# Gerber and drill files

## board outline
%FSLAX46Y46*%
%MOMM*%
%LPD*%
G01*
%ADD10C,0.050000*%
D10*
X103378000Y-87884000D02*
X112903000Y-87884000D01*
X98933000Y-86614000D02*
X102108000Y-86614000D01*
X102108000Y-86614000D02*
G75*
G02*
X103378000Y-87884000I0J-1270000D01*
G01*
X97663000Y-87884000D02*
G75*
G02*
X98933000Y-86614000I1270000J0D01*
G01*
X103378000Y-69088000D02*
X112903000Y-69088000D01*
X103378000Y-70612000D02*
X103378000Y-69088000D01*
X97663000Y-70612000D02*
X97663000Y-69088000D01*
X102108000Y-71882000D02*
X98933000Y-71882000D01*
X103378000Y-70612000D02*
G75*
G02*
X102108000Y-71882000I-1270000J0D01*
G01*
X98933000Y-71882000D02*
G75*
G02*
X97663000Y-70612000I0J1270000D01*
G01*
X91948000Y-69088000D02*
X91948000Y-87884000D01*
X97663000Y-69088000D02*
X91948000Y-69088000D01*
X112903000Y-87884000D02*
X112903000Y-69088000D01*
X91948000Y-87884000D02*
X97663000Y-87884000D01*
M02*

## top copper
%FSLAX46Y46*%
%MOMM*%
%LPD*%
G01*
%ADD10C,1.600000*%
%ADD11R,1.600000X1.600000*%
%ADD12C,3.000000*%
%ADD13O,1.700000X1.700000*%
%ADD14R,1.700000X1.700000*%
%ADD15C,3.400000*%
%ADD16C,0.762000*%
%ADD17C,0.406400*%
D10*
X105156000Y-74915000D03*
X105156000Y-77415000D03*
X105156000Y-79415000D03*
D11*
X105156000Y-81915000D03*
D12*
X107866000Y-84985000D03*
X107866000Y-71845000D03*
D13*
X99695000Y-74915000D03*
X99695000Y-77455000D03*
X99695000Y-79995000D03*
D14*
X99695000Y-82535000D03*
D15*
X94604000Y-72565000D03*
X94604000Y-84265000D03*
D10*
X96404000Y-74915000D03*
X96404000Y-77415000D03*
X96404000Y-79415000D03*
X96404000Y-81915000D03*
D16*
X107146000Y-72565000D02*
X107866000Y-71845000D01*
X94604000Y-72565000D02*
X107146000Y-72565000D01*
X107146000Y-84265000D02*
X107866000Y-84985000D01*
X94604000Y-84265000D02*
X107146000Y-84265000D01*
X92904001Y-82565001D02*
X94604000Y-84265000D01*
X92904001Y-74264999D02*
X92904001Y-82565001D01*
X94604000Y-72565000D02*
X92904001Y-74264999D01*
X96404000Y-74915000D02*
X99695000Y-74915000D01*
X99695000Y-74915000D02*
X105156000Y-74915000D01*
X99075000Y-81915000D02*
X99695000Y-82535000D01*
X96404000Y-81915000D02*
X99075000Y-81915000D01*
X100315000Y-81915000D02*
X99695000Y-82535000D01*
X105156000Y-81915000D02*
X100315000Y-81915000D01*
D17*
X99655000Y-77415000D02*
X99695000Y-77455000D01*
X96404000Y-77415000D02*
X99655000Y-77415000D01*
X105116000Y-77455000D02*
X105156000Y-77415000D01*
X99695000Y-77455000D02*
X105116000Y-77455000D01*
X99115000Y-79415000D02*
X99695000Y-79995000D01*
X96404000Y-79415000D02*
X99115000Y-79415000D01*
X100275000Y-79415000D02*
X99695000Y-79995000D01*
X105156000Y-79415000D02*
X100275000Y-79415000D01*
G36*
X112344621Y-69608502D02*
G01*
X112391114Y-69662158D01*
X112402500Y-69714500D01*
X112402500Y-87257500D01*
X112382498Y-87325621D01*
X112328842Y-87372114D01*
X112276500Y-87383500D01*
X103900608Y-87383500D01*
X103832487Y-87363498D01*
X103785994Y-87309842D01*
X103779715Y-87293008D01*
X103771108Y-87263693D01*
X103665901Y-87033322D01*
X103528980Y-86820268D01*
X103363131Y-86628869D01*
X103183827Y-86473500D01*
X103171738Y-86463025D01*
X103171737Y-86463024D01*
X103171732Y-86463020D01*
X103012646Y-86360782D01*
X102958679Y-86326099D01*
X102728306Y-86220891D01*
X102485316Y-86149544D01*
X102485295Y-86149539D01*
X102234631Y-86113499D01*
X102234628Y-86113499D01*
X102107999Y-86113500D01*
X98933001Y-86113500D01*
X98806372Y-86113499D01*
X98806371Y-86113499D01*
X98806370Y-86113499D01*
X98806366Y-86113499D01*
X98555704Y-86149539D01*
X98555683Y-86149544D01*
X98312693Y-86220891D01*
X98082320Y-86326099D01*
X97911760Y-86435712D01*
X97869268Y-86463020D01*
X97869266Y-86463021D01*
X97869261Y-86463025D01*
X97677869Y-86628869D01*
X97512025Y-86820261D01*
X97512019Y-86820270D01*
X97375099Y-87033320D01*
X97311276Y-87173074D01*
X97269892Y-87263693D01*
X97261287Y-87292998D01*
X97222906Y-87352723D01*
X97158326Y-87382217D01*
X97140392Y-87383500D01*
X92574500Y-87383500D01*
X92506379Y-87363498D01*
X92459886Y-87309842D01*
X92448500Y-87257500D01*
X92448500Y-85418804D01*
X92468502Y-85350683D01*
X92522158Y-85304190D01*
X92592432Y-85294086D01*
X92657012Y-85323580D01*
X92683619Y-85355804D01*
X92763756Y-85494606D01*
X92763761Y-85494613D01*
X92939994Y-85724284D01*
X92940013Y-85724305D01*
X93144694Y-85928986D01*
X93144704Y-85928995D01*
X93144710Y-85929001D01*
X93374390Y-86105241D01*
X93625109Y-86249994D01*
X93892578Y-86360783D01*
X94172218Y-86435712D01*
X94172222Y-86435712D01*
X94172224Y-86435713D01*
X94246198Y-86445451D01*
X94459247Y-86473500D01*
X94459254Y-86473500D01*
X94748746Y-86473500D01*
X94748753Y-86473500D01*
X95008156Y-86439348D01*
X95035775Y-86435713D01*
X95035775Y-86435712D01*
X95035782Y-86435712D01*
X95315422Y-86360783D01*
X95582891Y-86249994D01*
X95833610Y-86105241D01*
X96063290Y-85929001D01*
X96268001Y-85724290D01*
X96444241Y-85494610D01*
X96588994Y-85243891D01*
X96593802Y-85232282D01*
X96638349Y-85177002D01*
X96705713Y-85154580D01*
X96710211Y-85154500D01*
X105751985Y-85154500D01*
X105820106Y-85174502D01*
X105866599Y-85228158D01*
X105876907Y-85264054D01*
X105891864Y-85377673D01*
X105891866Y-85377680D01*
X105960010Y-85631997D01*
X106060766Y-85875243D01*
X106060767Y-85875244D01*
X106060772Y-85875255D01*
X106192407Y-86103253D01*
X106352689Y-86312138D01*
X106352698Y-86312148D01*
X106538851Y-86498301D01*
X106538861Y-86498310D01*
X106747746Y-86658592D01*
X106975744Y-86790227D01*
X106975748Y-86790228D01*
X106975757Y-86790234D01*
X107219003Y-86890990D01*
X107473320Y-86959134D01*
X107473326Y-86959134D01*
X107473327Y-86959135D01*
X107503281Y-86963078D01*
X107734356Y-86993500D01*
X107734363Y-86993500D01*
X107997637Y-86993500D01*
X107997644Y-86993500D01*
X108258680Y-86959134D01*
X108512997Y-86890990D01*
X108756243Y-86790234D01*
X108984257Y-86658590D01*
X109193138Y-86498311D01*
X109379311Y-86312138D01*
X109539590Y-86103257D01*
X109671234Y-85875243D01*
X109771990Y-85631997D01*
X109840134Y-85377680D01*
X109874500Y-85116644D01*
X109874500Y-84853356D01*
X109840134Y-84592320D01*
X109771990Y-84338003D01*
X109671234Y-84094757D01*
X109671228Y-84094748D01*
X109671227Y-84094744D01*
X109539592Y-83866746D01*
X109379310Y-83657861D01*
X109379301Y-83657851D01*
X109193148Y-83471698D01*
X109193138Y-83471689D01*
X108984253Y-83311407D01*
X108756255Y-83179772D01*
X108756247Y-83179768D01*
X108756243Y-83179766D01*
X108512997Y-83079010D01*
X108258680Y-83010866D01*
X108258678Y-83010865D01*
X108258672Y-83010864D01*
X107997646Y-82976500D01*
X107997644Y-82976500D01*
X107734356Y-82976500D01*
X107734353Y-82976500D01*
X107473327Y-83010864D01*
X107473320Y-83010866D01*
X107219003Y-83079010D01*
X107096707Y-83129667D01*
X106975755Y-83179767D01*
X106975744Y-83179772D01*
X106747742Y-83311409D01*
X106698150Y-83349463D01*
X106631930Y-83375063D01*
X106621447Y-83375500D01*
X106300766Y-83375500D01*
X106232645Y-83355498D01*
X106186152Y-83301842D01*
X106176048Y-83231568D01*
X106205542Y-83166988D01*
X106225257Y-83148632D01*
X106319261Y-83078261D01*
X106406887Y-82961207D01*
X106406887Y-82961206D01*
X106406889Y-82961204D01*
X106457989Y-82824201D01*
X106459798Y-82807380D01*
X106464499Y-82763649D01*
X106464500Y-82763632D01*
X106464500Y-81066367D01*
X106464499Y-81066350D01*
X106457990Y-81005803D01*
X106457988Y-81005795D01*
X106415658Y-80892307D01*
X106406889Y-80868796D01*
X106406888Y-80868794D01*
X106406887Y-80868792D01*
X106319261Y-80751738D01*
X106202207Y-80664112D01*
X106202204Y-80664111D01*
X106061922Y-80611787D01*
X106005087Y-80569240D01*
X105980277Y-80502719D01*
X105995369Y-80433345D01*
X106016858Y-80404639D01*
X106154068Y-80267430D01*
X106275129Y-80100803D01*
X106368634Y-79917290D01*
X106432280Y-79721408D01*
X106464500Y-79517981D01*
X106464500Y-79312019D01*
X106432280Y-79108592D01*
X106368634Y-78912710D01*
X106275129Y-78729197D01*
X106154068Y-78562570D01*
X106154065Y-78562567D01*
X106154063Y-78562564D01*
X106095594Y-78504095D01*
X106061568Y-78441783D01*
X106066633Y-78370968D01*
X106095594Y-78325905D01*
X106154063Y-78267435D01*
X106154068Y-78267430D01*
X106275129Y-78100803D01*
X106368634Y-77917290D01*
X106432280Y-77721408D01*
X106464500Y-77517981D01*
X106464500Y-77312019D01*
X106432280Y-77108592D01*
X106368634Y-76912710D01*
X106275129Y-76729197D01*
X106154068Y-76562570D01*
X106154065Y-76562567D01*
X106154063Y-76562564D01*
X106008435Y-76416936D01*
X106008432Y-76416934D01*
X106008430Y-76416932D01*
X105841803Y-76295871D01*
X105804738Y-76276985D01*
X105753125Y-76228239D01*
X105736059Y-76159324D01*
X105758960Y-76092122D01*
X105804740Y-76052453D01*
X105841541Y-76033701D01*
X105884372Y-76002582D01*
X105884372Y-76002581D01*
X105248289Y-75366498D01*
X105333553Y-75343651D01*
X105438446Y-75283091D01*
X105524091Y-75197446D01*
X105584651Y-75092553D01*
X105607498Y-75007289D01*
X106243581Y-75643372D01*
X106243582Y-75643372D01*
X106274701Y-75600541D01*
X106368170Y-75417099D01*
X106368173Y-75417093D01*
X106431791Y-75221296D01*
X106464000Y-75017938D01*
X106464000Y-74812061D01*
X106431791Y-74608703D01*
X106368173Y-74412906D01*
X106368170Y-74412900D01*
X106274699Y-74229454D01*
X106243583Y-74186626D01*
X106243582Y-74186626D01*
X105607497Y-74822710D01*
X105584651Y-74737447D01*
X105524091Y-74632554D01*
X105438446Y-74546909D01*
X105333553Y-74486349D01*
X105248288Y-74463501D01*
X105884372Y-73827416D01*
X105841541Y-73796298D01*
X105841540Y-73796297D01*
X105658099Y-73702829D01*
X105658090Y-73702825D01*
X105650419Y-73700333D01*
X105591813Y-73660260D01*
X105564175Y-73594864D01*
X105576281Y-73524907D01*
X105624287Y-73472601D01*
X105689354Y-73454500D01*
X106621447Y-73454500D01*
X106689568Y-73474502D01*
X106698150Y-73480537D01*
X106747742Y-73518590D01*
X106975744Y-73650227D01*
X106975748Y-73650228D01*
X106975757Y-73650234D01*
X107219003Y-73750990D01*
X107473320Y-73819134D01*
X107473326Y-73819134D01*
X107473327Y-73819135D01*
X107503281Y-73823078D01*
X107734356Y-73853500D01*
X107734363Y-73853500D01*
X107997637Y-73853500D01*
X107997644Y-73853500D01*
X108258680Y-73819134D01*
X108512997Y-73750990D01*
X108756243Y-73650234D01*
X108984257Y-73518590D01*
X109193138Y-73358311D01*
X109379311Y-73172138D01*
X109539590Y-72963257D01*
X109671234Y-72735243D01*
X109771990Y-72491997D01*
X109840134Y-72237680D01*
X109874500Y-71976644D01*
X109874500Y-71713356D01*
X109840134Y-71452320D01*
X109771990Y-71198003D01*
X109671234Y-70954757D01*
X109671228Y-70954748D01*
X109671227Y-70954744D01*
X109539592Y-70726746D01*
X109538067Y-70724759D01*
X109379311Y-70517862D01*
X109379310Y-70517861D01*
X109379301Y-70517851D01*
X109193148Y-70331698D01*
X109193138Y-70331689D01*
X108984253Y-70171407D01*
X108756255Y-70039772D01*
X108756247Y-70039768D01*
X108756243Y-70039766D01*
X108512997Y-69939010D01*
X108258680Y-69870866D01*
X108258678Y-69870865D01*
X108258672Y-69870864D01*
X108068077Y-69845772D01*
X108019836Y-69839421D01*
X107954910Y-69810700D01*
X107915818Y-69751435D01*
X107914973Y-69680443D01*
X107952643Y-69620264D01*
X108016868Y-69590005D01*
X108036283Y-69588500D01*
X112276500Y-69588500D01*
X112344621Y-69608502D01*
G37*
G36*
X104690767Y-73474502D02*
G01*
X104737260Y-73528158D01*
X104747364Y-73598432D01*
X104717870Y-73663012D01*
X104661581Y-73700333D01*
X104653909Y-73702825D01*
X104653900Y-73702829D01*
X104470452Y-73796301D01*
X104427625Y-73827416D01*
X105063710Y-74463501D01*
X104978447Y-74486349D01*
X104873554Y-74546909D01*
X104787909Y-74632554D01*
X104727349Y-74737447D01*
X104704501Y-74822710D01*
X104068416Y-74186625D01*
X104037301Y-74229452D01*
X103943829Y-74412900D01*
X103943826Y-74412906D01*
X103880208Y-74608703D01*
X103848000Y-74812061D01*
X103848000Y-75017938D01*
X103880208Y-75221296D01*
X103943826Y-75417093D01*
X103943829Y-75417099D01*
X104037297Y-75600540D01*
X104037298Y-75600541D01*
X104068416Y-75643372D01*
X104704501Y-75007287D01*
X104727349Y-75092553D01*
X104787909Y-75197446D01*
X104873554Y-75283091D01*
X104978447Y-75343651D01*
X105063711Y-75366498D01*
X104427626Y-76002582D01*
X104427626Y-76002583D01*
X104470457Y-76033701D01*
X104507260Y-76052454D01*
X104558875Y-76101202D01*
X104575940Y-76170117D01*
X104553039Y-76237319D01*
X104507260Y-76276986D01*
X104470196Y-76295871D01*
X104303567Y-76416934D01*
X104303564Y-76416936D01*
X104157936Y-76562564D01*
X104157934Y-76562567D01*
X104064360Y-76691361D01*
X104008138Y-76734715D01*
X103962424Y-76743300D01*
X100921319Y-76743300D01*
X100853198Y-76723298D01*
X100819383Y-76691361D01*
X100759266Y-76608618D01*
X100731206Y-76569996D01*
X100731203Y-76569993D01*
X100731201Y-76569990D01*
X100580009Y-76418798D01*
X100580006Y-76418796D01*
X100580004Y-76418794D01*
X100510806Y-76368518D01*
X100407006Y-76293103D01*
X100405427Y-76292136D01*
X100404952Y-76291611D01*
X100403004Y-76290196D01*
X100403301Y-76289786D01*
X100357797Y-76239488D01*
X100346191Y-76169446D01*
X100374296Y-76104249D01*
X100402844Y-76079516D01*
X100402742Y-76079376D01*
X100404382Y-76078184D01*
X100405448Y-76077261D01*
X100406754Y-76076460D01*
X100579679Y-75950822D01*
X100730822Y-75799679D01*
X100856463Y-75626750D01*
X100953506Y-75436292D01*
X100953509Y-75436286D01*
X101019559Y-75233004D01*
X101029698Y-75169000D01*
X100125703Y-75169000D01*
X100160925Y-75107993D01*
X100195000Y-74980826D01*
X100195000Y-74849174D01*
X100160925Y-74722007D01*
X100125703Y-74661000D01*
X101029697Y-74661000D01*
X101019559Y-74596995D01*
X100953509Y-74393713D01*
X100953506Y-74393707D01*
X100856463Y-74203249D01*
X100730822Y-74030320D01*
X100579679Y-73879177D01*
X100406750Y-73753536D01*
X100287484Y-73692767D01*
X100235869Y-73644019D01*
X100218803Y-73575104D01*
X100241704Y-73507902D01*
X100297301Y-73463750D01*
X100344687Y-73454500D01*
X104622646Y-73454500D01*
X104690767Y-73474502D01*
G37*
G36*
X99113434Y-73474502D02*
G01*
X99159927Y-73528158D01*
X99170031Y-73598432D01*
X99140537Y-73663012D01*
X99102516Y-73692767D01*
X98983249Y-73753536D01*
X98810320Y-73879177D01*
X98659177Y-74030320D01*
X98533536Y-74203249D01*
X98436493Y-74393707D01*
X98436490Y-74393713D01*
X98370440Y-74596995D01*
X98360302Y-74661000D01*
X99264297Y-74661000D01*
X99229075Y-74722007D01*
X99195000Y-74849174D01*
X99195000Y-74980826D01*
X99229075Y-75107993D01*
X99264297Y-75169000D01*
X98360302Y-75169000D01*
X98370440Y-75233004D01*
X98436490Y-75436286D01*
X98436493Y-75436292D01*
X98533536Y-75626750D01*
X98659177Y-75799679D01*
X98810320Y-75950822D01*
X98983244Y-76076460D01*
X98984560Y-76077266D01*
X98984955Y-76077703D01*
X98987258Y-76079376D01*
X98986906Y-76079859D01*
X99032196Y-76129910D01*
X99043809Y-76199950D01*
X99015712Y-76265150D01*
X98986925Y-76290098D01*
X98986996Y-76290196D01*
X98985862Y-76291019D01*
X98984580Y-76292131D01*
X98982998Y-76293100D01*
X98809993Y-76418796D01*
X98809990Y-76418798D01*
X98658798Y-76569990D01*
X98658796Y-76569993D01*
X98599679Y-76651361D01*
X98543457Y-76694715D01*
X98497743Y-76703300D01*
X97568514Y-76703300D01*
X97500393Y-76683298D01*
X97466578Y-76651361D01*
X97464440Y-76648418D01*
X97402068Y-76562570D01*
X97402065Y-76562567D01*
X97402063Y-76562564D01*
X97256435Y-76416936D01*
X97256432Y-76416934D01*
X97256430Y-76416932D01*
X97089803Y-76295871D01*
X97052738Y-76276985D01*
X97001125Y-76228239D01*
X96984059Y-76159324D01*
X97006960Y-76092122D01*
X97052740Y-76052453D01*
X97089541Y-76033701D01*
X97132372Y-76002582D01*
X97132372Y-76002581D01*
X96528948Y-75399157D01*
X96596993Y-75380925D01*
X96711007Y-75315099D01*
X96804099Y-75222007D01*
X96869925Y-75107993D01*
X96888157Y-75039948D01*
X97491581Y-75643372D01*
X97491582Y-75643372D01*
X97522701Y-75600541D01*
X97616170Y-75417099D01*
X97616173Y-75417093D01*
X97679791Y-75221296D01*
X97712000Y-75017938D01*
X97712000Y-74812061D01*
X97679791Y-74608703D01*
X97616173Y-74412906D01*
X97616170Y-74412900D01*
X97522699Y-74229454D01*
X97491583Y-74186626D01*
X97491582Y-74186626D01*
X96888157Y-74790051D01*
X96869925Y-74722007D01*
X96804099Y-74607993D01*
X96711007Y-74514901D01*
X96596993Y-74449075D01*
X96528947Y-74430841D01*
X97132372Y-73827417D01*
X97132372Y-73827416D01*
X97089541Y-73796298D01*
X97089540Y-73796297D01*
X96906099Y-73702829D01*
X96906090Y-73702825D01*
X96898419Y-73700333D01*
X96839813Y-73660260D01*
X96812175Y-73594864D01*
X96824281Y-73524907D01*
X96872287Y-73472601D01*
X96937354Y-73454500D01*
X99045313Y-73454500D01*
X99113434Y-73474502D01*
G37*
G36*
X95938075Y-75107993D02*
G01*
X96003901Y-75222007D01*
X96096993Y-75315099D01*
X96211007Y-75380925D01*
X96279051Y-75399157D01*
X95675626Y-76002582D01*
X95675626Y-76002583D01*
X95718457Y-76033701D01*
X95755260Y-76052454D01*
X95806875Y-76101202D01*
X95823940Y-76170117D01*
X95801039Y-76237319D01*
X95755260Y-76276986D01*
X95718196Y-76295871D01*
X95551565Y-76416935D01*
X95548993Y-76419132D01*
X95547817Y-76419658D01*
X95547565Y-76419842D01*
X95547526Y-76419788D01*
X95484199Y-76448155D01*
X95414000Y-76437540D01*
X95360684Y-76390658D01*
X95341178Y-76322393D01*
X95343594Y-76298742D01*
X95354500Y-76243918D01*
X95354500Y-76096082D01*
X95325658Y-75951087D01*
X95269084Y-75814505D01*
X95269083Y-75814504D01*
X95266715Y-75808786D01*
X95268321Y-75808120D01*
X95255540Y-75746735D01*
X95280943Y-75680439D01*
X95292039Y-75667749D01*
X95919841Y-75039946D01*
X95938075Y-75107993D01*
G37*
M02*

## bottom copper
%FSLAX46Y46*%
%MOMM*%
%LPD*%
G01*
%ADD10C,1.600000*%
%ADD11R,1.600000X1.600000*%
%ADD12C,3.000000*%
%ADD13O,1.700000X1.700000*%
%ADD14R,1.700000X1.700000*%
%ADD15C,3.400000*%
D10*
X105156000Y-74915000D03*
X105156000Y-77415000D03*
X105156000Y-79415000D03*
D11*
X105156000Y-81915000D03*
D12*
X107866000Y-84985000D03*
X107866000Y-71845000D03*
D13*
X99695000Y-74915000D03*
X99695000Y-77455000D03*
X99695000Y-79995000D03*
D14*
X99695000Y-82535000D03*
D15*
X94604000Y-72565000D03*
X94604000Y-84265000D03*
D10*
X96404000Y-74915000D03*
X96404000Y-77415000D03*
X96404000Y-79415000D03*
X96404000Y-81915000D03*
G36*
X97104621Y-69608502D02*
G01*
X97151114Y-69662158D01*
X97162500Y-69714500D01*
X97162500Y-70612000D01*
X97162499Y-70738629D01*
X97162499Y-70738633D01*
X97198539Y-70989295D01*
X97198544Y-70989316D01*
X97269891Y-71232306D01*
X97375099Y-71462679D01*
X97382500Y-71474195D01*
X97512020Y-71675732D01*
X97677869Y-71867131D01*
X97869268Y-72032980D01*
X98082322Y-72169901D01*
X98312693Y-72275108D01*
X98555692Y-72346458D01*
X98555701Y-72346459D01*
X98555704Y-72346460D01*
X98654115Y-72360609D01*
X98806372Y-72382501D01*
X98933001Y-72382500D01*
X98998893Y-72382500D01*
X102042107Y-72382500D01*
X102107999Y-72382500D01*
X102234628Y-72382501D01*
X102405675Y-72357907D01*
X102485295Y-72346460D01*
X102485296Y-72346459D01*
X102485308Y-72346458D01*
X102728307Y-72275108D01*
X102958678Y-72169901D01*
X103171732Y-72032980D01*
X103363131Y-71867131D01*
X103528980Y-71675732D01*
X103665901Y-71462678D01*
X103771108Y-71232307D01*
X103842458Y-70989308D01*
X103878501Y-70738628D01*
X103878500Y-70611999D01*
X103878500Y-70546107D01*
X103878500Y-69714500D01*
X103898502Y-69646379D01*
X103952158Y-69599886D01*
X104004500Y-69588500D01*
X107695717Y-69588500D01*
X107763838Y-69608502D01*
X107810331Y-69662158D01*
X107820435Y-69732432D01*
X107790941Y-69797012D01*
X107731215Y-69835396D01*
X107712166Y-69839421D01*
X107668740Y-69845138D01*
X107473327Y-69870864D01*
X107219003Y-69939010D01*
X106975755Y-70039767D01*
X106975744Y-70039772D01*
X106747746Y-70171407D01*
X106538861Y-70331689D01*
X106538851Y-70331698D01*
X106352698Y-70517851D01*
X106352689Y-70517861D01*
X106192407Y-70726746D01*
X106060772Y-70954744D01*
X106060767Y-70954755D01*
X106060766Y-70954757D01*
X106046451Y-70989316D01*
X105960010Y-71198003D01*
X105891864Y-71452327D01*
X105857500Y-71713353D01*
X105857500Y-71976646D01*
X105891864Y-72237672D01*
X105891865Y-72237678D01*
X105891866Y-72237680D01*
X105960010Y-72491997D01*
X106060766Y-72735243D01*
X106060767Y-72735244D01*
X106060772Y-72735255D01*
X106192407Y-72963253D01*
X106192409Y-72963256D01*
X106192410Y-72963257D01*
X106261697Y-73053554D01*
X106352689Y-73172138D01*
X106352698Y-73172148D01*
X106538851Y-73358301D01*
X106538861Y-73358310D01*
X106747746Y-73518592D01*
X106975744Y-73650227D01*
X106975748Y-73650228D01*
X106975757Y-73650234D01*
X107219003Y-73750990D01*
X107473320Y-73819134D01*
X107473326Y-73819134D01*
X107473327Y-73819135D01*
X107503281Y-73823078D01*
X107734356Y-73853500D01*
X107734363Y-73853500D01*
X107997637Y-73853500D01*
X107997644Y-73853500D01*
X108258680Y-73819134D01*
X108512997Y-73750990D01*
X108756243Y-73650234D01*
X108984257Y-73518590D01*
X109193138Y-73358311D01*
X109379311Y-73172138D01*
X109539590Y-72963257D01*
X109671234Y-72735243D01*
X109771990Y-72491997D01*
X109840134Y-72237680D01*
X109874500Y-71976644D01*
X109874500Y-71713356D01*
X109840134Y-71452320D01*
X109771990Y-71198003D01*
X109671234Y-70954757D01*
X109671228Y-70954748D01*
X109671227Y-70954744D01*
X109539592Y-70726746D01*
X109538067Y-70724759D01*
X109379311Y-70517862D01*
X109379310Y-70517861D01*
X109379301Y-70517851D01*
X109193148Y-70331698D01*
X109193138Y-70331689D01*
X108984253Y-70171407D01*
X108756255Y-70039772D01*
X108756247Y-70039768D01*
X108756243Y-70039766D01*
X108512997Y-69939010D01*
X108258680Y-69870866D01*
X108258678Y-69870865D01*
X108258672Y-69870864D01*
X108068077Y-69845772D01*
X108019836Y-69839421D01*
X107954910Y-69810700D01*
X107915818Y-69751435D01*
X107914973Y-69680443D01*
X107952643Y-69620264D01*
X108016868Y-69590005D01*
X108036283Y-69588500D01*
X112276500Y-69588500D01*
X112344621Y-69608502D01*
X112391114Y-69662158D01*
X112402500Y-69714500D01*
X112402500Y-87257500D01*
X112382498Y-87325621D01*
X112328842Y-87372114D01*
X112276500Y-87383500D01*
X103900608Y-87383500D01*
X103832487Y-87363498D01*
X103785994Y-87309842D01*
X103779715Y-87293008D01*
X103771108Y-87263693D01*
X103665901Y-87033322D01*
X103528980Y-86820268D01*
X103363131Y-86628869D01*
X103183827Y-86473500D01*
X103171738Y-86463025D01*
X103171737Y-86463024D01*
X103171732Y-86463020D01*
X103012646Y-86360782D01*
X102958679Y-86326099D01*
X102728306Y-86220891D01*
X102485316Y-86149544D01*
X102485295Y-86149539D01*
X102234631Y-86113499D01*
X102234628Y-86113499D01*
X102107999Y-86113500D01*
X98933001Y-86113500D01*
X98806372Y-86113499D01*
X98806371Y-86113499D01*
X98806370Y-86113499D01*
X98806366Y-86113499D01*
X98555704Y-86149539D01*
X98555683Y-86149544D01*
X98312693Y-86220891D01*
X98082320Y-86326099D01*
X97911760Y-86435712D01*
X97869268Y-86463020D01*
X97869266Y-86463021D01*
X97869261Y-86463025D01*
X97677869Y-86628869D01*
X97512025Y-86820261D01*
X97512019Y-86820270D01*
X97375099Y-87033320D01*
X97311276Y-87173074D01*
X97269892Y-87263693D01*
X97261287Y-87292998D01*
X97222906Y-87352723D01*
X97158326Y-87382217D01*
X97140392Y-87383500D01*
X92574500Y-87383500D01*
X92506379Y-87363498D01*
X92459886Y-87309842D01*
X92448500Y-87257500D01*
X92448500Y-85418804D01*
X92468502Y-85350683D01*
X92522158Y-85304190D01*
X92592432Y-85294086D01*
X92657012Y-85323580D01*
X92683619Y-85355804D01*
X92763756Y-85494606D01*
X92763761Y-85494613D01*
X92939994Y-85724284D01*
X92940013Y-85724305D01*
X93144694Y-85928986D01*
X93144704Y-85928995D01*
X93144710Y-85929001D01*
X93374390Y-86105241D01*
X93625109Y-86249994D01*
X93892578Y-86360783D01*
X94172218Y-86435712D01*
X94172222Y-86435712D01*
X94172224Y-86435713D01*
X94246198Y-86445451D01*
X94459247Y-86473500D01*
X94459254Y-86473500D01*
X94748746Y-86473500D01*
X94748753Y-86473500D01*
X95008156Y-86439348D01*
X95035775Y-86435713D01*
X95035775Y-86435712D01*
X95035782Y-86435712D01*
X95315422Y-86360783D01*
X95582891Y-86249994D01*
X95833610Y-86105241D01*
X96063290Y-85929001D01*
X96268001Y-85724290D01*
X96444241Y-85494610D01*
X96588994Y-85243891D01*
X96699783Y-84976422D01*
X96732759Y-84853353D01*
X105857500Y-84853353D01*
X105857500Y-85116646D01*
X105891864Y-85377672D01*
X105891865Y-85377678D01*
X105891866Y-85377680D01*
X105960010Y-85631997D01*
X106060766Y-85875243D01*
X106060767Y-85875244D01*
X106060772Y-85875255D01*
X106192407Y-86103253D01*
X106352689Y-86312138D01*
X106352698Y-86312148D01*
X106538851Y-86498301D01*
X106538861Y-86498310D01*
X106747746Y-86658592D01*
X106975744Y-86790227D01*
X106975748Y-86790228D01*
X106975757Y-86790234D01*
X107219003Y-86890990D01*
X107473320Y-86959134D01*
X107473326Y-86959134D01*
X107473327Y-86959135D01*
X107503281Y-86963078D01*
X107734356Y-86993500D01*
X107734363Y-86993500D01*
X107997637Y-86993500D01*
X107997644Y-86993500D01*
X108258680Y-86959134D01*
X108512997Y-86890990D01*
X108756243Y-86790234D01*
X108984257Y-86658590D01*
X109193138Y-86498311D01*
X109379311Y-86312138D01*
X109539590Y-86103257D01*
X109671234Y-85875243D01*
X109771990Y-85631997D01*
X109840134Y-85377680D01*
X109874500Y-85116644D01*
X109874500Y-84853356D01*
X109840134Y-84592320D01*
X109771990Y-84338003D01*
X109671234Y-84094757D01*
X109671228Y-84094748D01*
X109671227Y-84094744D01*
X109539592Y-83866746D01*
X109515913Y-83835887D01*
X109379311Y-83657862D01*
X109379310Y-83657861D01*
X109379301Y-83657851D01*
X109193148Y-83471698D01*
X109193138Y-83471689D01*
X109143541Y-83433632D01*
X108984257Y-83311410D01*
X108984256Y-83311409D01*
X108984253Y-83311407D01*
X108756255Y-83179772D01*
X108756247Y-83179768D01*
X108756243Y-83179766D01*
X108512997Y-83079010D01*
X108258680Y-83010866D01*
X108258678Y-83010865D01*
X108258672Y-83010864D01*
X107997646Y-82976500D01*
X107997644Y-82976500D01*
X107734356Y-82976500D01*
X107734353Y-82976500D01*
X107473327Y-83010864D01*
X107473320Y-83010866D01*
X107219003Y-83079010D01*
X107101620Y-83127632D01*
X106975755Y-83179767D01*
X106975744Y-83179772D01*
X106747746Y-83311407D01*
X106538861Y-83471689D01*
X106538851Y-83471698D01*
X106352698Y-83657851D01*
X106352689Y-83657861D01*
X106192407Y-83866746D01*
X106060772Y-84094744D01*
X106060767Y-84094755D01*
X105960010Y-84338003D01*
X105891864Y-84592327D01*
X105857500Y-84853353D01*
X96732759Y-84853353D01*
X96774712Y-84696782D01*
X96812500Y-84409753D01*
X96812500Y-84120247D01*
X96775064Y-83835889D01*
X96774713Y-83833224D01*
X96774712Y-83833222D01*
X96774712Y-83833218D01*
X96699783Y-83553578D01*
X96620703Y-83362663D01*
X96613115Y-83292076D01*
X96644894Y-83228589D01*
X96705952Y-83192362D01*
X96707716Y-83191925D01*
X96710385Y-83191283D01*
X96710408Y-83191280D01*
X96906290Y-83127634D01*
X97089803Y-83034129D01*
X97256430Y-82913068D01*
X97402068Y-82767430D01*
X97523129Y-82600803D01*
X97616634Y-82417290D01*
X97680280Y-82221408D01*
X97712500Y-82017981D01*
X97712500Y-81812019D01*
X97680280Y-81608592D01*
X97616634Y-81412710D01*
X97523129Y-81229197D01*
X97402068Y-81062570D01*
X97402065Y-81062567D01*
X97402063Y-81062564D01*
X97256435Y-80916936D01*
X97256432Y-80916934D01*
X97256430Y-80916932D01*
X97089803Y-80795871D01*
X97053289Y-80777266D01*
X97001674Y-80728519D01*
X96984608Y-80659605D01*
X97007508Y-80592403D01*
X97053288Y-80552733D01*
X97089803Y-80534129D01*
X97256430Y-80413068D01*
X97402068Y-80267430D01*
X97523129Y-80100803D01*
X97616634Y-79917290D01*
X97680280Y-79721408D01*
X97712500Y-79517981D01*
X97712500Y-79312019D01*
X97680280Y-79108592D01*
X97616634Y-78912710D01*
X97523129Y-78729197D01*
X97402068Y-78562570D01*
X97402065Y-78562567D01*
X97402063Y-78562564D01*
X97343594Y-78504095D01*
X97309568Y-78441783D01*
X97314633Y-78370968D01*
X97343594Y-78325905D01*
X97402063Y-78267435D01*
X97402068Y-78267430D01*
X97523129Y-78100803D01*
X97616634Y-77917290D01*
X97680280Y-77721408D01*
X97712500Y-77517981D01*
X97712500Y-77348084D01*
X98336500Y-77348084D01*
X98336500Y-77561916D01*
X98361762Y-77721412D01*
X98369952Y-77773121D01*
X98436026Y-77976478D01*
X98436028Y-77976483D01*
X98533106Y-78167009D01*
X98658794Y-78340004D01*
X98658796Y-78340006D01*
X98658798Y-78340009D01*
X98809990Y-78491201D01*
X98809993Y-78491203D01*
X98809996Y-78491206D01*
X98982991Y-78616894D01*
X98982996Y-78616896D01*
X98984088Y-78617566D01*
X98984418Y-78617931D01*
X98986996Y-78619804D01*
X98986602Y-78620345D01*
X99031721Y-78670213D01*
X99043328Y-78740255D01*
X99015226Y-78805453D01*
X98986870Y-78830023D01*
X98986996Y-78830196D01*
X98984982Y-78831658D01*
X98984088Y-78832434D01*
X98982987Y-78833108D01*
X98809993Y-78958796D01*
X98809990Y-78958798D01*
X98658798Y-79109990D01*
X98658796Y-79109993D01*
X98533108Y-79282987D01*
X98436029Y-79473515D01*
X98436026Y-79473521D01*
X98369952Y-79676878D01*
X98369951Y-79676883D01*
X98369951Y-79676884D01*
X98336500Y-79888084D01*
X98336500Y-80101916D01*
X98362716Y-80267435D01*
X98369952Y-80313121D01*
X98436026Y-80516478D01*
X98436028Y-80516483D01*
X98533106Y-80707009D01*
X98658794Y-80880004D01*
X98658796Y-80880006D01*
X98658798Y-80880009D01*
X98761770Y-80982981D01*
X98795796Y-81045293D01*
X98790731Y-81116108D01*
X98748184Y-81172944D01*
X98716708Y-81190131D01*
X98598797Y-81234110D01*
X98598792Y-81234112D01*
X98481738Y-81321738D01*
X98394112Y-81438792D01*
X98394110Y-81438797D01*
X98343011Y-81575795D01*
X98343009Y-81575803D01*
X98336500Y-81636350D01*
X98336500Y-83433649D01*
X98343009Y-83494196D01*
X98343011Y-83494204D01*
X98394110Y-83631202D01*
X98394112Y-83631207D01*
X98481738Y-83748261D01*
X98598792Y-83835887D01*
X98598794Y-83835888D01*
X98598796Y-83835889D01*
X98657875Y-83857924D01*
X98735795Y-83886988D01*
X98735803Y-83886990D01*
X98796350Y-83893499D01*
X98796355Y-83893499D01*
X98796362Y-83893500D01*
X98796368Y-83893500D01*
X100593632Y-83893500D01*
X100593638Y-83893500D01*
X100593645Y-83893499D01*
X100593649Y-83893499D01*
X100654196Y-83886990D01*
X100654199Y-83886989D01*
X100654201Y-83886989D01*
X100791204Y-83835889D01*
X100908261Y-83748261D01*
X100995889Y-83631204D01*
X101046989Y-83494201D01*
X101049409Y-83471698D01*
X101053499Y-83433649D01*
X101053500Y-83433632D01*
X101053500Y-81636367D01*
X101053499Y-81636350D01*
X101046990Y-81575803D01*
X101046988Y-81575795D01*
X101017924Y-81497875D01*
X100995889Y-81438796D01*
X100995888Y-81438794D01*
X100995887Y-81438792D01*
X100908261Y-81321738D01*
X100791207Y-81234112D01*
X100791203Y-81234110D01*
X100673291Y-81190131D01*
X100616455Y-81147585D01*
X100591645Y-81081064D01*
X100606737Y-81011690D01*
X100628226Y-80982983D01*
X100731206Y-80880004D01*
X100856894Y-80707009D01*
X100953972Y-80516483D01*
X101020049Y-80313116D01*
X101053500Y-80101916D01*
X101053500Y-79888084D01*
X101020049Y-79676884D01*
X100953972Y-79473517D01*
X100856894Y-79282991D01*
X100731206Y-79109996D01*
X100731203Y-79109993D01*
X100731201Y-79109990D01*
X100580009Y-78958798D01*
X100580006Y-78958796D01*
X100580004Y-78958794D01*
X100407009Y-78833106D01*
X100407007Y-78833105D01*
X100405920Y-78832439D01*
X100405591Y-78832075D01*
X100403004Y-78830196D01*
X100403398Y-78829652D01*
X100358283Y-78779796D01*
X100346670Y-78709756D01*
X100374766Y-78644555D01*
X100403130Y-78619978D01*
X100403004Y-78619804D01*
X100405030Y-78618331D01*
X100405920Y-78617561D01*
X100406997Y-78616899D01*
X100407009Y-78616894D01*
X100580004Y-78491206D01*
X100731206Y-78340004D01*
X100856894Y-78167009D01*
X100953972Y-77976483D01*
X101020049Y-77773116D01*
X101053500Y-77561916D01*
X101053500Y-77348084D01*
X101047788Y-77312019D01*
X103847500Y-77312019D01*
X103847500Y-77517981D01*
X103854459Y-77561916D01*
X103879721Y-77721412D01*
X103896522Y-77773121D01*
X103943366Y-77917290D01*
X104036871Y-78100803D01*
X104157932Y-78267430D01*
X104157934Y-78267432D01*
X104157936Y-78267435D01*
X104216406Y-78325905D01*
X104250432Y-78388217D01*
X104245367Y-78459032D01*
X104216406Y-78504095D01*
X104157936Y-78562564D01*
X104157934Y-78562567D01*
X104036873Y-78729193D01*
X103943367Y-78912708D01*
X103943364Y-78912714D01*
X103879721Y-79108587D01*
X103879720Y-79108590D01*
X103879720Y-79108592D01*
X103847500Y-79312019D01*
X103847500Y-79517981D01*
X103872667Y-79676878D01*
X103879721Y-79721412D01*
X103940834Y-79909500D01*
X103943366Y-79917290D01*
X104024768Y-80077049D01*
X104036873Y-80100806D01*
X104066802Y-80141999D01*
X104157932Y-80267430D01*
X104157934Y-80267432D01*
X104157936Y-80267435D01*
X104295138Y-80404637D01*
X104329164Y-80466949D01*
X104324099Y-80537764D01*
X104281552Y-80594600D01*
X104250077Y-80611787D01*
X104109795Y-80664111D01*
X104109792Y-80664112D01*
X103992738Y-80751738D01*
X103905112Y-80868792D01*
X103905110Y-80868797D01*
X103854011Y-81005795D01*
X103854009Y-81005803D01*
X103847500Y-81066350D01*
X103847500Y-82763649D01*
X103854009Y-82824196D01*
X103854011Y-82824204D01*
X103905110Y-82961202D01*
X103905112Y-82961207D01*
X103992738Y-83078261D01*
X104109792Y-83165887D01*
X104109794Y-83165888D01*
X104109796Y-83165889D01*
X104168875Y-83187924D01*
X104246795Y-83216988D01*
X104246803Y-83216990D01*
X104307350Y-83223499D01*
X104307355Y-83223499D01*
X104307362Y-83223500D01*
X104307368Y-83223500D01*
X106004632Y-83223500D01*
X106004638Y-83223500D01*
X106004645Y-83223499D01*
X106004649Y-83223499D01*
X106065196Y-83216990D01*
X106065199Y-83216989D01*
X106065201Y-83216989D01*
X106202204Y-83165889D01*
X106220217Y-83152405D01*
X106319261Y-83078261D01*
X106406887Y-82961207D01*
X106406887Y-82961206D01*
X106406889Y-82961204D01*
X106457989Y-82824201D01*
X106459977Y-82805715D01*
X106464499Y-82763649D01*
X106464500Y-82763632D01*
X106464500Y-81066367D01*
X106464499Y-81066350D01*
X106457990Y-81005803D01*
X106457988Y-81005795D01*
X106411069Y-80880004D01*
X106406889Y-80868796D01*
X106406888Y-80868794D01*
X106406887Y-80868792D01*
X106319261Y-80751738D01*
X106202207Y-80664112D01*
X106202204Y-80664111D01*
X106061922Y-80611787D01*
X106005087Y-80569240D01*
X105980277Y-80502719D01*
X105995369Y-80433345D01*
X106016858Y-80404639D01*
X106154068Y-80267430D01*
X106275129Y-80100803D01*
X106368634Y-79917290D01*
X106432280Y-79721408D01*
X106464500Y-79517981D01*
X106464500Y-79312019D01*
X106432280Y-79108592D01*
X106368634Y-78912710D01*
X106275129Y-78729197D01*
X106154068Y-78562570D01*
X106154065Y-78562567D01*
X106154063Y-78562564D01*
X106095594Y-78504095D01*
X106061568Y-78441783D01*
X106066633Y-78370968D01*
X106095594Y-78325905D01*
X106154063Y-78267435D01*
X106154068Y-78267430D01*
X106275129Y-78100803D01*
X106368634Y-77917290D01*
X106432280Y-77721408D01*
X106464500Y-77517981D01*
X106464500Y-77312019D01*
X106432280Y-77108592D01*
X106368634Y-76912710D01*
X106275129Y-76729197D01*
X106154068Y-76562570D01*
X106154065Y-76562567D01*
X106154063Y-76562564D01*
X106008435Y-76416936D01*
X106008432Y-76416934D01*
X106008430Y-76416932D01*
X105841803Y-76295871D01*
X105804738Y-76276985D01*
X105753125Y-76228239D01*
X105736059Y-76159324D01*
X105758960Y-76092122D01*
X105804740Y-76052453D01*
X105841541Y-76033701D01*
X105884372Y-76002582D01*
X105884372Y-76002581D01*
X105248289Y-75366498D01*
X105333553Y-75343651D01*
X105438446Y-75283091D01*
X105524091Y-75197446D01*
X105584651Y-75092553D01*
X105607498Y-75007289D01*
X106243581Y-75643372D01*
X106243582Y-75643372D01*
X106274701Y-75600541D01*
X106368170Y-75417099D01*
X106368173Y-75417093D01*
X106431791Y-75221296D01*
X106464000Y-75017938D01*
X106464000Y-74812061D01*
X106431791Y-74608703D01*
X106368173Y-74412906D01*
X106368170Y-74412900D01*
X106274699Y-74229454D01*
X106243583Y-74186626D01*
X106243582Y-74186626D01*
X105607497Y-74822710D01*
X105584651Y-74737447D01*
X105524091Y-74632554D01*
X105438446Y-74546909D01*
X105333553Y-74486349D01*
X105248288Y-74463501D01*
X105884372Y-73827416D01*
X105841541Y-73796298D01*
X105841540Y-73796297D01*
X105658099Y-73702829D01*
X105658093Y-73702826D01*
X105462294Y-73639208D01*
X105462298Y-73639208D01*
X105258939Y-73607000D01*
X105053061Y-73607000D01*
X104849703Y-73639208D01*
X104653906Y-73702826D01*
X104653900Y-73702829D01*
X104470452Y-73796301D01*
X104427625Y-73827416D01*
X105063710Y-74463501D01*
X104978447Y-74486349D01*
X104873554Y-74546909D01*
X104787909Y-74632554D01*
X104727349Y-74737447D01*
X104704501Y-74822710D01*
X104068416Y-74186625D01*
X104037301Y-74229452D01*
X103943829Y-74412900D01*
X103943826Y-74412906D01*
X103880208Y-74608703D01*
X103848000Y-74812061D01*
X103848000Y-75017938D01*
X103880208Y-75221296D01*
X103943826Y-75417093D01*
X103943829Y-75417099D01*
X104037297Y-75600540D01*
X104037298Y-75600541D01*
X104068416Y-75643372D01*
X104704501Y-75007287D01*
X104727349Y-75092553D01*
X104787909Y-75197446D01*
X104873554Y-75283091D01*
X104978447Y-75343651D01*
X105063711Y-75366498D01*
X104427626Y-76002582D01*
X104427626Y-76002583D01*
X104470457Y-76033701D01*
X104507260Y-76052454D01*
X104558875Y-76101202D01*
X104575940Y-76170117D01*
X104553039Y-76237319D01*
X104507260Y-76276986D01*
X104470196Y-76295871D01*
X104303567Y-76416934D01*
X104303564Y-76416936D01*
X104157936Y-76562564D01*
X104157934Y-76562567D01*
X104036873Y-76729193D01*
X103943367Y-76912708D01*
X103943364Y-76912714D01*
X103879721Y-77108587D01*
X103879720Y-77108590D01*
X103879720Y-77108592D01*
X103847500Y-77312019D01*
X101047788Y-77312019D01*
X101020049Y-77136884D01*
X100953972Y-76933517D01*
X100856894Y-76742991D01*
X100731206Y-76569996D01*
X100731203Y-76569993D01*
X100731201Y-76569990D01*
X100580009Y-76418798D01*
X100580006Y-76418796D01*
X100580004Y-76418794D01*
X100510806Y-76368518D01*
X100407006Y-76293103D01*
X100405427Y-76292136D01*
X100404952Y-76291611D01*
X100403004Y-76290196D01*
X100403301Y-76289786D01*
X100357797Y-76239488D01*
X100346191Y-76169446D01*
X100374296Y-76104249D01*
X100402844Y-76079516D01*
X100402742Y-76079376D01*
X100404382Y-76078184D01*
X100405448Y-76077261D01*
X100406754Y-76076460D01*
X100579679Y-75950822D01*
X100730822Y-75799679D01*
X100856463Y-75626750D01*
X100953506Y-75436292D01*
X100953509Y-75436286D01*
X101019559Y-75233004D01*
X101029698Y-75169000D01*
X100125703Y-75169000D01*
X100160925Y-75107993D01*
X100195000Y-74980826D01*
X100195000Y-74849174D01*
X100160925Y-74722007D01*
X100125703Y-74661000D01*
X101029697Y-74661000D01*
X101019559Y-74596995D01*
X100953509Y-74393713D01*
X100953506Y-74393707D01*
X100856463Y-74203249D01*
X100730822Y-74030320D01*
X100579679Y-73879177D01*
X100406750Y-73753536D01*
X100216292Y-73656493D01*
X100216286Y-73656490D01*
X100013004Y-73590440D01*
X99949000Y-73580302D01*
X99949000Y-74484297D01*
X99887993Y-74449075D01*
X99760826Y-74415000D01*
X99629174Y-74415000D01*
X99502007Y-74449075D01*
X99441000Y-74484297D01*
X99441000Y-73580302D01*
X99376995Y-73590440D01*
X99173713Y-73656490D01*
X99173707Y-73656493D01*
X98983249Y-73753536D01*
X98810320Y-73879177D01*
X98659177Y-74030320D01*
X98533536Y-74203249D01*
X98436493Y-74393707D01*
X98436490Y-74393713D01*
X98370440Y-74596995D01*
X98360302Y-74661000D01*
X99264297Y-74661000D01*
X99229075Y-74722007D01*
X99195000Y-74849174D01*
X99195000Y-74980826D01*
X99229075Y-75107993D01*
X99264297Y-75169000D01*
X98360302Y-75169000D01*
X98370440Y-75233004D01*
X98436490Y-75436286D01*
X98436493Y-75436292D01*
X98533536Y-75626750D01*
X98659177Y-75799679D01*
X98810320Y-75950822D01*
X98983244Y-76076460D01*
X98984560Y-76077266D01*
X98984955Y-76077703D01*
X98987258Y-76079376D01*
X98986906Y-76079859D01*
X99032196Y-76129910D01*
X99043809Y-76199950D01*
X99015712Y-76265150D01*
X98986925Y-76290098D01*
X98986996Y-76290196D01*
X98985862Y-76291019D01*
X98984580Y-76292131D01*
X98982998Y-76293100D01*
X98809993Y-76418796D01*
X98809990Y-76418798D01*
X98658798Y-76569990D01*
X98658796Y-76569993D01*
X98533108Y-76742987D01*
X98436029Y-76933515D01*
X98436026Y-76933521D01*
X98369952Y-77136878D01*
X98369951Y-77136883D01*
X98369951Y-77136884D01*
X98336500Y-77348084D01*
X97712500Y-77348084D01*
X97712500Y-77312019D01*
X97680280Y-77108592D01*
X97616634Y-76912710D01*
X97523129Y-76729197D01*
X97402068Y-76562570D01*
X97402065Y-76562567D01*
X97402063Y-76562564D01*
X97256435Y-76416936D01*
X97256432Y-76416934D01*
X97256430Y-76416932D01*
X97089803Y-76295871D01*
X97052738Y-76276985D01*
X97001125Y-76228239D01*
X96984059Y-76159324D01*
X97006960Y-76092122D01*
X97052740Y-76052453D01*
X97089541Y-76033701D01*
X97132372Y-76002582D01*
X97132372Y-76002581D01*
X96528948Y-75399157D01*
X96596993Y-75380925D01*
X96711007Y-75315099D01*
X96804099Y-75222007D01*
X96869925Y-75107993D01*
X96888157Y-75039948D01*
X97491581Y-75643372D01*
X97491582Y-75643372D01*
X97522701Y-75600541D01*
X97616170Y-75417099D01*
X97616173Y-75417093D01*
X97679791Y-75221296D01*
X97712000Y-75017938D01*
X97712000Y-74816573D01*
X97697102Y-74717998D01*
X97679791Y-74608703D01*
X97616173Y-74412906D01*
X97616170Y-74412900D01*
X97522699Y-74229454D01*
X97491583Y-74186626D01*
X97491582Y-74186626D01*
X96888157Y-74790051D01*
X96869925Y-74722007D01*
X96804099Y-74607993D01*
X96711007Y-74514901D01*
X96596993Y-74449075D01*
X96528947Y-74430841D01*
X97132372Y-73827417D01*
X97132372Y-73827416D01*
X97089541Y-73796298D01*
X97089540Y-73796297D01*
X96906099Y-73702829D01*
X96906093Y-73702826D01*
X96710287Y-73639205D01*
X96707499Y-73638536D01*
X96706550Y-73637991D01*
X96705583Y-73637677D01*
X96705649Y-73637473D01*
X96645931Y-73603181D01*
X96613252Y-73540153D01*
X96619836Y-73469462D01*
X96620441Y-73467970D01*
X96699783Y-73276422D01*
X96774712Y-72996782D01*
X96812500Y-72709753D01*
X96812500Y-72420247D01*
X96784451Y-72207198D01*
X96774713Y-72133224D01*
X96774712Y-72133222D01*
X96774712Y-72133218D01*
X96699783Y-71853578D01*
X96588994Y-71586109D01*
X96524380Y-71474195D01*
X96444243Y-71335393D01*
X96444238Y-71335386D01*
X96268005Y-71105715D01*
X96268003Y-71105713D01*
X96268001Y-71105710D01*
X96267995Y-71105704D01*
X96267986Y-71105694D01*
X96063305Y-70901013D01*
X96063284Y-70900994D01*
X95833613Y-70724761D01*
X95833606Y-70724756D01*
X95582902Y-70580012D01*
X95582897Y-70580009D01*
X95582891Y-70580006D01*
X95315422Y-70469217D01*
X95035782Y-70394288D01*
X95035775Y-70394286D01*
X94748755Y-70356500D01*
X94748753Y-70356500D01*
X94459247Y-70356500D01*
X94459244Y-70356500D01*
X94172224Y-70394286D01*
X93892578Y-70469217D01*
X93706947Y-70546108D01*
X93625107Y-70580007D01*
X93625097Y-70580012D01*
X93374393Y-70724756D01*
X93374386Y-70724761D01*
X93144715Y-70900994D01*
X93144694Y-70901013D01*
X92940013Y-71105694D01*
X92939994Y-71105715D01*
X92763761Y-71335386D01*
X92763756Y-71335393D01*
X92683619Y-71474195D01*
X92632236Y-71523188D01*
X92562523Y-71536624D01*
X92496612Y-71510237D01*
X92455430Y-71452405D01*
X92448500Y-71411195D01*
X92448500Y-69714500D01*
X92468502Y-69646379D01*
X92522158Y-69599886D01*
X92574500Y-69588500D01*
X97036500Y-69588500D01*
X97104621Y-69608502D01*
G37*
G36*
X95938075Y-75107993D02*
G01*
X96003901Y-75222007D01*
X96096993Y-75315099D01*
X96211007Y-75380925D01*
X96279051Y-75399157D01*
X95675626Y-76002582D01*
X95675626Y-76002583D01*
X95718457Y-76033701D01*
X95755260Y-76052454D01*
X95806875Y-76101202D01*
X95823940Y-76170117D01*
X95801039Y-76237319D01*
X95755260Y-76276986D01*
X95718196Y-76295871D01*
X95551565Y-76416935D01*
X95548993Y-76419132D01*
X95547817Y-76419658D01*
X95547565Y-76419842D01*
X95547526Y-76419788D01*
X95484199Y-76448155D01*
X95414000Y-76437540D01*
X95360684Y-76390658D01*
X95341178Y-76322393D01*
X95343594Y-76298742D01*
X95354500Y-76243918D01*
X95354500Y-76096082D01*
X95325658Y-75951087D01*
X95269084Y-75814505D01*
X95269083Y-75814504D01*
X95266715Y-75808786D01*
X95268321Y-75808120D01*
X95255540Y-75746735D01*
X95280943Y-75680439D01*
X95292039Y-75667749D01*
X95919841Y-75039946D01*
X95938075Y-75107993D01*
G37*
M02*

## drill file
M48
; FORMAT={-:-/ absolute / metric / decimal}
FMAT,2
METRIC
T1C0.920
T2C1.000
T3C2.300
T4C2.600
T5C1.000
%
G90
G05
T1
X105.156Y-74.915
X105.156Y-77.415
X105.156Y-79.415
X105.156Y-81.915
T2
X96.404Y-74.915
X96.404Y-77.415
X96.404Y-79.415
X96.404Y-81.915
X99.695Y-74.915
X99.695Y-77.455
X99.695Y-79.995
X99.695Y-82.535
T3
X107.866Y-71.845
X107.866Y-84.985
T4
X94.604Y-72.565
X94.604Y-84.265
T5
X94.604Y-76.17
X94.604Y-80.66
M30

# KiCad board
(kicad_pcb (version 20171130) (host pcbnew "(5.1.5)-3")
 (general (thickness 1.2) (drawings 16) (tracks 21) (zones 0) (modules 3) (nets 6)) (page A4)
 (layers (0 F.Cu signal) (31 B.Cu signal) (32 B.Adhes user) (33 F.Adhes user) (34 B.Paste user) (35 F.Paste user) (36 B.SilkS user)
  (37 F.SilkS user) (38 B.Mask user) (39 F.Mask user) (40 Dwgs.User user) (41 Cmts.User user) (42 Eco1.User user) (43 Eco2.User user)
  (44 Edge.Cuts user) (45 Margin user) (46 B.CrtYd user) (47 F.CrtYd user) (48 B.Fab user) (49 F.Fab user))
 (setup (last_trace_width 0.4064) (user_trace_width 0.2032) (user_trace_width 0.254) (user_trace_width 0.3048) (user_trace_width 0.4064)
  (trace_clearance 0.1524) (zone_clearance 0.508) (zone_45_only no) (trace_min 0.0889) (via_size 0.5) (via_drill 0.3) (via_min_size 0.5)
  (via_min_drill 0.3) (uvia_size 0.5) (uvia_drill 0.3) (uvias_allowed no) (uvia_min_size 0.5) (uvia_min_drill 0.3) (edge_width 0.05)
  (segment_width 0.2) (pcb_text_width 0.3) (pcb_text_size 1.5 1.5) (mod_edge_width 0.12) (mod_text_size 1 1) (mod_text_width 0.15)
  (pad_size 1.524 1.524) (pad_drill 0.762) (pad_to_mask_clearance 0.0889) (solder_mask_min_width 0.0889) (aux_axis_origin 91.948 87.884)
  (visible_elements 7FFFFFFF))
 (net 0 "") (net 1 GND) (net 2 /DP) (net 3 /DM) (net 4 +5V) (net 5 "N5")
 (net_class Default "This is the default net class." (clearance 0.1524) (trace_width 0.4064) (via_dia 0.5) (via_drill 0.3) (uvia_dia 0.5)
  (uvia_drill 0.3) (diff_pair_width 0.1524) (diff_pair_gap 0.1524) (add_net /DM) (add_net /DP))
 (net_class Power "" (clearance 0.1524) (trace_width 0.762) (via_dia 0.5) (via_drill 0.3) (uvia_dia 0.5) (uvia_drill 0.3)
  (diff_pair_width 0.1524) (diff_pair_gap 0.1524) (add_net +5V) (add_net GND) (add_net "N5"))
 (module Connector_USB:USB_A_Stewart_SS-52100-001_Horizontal (layer F.Cu) (at 105.156 81.915 90)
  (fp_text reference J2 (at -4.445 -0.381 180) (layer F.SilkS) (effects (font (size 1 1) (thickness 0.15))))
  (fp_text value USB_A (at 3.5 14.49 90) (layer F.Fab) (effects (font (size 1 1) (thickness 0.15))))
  (pad 4 thru_hole circle (at 7 0 90) (size 1.6 1.6) (drill 0.92) (layers *.Cu *.Mask) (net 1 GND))
  (pad 3 thru_hole circle (at 4.5 0 90) (size 1.6 1.6) (drill 0.92) (layers *.Cu *.Mask) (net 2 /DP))
  (pad 2 thru_hole circle (at 2.5 0 90) (size 1.6 1.6) (drill 0.92) (layers *.Cu *.Mask) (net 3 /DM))
  (pad 1 thru_hole rect (at 0 0 90) (size 1.6 1.6) (drill 0.92) (layers *.Cu *.Mask) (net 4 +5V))
  (pad 5 thru_hole circle (at -3.07 2.71 90) (size 3 3) (drill 2.3) (layers *.Cu *.Mask) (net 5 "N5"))
  (pad 5 thru_hole circle (at 10.07 2.71 90) (size 3 3) (drill 2.3) (layers *.Cu *.Mask) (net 5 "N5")))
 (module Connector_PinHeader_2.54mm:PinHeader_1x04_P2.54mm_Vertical (layer F.Cu) (at 99.695 82.535 180)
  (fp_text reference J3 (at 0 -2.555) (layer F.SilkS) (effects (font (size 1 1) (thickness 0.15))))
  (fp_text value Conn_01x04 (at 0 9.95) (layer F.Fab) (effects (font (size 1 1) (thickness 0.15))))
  (pad 4 thru_hole oval (at 0 7.62 180) (size 1.7 1.7) (drill 1) (layers *.Cu *.Mask) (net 1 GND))
  (pad 3 thru_hole oval (at 0 5.08 180) (size 1.7 1.7) (drill 1) (layers *.Cu *.Mask) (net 2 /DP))
  (pad 2 thru_hole oval (at 0 2.54 180) (size 1.7 1.7) (drill 1) (layers *.Cu *.Mask) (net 3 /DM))
  (pad 1 thru_hole rect (at 0 0 180) (size 1.7 1.7) (drill 1) (layers *.Cu *.Mask) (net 4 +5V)))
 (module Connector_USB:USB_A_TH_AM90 (layer F.Cu) (at 95.504 78.415 270)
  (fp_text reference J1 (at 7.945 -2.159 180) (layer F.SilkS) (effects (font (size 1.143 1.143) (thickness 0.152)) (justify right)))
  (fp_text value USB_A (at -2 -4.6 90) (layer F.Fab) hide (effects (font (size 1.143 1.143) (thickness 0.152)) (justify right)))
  (pad 5 thru_hole circle (at -5.85 0.9 180) (size 3.4 3.4) (drill 2.6) (layers *.Cu *.Mask) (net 5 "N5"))
  (pad 5 thru_hole circle (at 5.85 0.9 180) (size 3.4 3.4) (drill 2.6) (layers *.Cu *.Mask) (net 5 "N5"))
  (pad 4 thru_hole circle (at -3.5 -0.9 180) (size 1.6 1.6) (drill 1) (layers *.Cu *.Mask) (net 1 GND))
  (pad 3 thru_hole circle (at -1 -0.9 180) (size 1.6 1.6) (drill 1) (layers *.Cu *.Mask) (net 2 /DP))
  (pad 2 thru_hole circle (at 1 -0.9 180) (size 1.6 1.6) (drill 1) (layers *.Cu *.Mask) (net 3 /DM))
  (pad 1 thru_hole circle (at 3.5 -0.9 180) (size 1.6 1.6) (drill 1) (layers *.Cu *.Mask) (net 4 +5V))
  (pad "" np_thru_hole circle (at -2.245 0.9 270) (size 1 1) (drill 1) (layers *.Cu *.Mask))
  (pad "" np_thru_hole circle (at 2.245 0.9 270) (size 1 1) (drill 1) (layers *.Cu *.Mask)))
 (gr_line (start 103.378 87.884) (end 112.903 87.884) (layer Edge.Cuts) (width 0.05))
 (gr_line (start 98.933 86.614) (end 102.108 86.614) (layer Edge.Cuts) (width 0.05))
 (gr_arc (start 102.108 87.884) (end 103.378 87.884) (angle -90) (layer Edge.Cuts) (width 0.05))
 (gr_arc (start 98.933 87.884) (end 98.933 86.614) (angle -90) (layer Edge.Cuts) (width 0.05))
 (gr_line (start 103.378 69.088) (end 112.903 69.088) (layer Edge.Cuts) (width 0.05))
 (gr_line (start 103.378 70.612) (end 103.378 69.088) (layer Edge.Cuts) (width 0.05))
 (gr_line (start 97.663 70.612) (end 97.663 69.088) (layer Edge.Cuts) (width 0.05))
 (gr_line (start 102.108 71.882) (end 98.933 71.882) (layer Edge.Cuts) (width 0.05))
 (gr_arc (start 102.108 70.612) (end 102.108 71.882) (angle -90) (layer Edge.Cuts) (width 0.05))
 (gr_arc (start 98.933 70.612) (end 97.663 70.612) (angle -90) (layer Edge.Cuts) (width 0.05))
 (gr_line (start 91.948 69.088) (end 91.948 87.884) (layer Edge.Cuts) (width 0.05))
 (gr_line (start 97.663 69.088) (end 91.948 69.088) (layer Edge.Cuts) (width 0.05))
 (gr_line (start 112.903 87.884) (end 112.903 69.088) (layer Edge.Cuts) (width 0.05))
 (gr_line (start 91.948 87.884) (end 97.663 87.884) (layer Edge.Cuts) (width 0.05))
 (segment (start 107.146 72.565) (end 107.866 71.845) (width 0.762) (layer F.Cu) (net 5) (status 30))
 (segment (start 94.604 72.565) (end 107.146 72.565) (width 0.762) (layer F.Cu) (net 5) (status 30))
 (segment (start 107.146 84.265) (end 107.866 84.985) (width 0.762) (layer F.Cu) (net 5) (status 30))
 (segment (start 94.604 84.265) (end 107.146 84.265) (width 0.762) (layer F.Cu) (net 5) (status 30))
 (segment (start 92.904001 82.565001) (end 94.604 84.265) (width 0.762) (layer F.Cu) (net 5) (status 20))
 (segment (start 92.904001 74.264999) (end 92.904001 82.565001) (width 0.762) (layer F.Cu) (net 5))
 (segment (start 94.604 72.565) (end 92.904001 74.264999) (width 0.762) (layer F.Cu) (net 5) (status 10))
 (segment (start 96.404 74.915) (end 99.695 74.915) (width 0.762) (layer F.Cu) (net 1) (status 30))
 (segment (start 99.695 74.915) (end 105.156 74.915) (width 0.762) (layer F.Cu) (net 1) (status 30))
 (segment (start 99.075 81.915) (end 99.695 82.535) (width 0.762) (layer F.Cu) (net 4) (status 30))
 (segment (start 96.404 81.915) (end 99.075 81.915) (width 0.762) (layer F.Cu) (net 4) (status 30))
 (segment (start 100.315 81.915) (end 99.695 82.535) (width 0.762) (layer F.Cu) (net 4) (status 30))
 (segment (start 105.156 81.915) (end 100.315 81.915) (width 0.762) (layer F.Cu) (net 4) (status 30))
 (segment (start 99.655 77.415) (end 99.695 77.455) (width 0.4064) (layer F.Cu) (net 2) (status 30))
 (segment (start 96.404 77.415) (end 99.655 77.415) (width 0.4064) (layer F.Cu) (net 2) (status 30))
 (segment (start 105.116 77.455) (end 105.156 77.415) (width 0.4064) (layer F.Cu) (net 2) (status 30))
 (segment (start 99.695 77.455) (end 105.116 77.455) (width 0.4064) (layer F.Cu) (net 2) (status 30))
 (segment (start 99.115 79.415) (end 99.695 79.995) (width 0.4064) (layer F.Cu) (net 3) (status 30))
 (segment (start 96.404 79.415) (end 99.115 79.415) (width 0.4064) (layer F.Cu) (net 3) (status 30))
 (segment (start 100.275 79.415) (end 99.695 79.995) (width 0.4064) (layer F.Cu) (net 3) (status 30))
 (segment (start 105.156 79.415) (end 100.275 79.415) (width 0.4064) (layer F.Cu) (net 3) (status 30))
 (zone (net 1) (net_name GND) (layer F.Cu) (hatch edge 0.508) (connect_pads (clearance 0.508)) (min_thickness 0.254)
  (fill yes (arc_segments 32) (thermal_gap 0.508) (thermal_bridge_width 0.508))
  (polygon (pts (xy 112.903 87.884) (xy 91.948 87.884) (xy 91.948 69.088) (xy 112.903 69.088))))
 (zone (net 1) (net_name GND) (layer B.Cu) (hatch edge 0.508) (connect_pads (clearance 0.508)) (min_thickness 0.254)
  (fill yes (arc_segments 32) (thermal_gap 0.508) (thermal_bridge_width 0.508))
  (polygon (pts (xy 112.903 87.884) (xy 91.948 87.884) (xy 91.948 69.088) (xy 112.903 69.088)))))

